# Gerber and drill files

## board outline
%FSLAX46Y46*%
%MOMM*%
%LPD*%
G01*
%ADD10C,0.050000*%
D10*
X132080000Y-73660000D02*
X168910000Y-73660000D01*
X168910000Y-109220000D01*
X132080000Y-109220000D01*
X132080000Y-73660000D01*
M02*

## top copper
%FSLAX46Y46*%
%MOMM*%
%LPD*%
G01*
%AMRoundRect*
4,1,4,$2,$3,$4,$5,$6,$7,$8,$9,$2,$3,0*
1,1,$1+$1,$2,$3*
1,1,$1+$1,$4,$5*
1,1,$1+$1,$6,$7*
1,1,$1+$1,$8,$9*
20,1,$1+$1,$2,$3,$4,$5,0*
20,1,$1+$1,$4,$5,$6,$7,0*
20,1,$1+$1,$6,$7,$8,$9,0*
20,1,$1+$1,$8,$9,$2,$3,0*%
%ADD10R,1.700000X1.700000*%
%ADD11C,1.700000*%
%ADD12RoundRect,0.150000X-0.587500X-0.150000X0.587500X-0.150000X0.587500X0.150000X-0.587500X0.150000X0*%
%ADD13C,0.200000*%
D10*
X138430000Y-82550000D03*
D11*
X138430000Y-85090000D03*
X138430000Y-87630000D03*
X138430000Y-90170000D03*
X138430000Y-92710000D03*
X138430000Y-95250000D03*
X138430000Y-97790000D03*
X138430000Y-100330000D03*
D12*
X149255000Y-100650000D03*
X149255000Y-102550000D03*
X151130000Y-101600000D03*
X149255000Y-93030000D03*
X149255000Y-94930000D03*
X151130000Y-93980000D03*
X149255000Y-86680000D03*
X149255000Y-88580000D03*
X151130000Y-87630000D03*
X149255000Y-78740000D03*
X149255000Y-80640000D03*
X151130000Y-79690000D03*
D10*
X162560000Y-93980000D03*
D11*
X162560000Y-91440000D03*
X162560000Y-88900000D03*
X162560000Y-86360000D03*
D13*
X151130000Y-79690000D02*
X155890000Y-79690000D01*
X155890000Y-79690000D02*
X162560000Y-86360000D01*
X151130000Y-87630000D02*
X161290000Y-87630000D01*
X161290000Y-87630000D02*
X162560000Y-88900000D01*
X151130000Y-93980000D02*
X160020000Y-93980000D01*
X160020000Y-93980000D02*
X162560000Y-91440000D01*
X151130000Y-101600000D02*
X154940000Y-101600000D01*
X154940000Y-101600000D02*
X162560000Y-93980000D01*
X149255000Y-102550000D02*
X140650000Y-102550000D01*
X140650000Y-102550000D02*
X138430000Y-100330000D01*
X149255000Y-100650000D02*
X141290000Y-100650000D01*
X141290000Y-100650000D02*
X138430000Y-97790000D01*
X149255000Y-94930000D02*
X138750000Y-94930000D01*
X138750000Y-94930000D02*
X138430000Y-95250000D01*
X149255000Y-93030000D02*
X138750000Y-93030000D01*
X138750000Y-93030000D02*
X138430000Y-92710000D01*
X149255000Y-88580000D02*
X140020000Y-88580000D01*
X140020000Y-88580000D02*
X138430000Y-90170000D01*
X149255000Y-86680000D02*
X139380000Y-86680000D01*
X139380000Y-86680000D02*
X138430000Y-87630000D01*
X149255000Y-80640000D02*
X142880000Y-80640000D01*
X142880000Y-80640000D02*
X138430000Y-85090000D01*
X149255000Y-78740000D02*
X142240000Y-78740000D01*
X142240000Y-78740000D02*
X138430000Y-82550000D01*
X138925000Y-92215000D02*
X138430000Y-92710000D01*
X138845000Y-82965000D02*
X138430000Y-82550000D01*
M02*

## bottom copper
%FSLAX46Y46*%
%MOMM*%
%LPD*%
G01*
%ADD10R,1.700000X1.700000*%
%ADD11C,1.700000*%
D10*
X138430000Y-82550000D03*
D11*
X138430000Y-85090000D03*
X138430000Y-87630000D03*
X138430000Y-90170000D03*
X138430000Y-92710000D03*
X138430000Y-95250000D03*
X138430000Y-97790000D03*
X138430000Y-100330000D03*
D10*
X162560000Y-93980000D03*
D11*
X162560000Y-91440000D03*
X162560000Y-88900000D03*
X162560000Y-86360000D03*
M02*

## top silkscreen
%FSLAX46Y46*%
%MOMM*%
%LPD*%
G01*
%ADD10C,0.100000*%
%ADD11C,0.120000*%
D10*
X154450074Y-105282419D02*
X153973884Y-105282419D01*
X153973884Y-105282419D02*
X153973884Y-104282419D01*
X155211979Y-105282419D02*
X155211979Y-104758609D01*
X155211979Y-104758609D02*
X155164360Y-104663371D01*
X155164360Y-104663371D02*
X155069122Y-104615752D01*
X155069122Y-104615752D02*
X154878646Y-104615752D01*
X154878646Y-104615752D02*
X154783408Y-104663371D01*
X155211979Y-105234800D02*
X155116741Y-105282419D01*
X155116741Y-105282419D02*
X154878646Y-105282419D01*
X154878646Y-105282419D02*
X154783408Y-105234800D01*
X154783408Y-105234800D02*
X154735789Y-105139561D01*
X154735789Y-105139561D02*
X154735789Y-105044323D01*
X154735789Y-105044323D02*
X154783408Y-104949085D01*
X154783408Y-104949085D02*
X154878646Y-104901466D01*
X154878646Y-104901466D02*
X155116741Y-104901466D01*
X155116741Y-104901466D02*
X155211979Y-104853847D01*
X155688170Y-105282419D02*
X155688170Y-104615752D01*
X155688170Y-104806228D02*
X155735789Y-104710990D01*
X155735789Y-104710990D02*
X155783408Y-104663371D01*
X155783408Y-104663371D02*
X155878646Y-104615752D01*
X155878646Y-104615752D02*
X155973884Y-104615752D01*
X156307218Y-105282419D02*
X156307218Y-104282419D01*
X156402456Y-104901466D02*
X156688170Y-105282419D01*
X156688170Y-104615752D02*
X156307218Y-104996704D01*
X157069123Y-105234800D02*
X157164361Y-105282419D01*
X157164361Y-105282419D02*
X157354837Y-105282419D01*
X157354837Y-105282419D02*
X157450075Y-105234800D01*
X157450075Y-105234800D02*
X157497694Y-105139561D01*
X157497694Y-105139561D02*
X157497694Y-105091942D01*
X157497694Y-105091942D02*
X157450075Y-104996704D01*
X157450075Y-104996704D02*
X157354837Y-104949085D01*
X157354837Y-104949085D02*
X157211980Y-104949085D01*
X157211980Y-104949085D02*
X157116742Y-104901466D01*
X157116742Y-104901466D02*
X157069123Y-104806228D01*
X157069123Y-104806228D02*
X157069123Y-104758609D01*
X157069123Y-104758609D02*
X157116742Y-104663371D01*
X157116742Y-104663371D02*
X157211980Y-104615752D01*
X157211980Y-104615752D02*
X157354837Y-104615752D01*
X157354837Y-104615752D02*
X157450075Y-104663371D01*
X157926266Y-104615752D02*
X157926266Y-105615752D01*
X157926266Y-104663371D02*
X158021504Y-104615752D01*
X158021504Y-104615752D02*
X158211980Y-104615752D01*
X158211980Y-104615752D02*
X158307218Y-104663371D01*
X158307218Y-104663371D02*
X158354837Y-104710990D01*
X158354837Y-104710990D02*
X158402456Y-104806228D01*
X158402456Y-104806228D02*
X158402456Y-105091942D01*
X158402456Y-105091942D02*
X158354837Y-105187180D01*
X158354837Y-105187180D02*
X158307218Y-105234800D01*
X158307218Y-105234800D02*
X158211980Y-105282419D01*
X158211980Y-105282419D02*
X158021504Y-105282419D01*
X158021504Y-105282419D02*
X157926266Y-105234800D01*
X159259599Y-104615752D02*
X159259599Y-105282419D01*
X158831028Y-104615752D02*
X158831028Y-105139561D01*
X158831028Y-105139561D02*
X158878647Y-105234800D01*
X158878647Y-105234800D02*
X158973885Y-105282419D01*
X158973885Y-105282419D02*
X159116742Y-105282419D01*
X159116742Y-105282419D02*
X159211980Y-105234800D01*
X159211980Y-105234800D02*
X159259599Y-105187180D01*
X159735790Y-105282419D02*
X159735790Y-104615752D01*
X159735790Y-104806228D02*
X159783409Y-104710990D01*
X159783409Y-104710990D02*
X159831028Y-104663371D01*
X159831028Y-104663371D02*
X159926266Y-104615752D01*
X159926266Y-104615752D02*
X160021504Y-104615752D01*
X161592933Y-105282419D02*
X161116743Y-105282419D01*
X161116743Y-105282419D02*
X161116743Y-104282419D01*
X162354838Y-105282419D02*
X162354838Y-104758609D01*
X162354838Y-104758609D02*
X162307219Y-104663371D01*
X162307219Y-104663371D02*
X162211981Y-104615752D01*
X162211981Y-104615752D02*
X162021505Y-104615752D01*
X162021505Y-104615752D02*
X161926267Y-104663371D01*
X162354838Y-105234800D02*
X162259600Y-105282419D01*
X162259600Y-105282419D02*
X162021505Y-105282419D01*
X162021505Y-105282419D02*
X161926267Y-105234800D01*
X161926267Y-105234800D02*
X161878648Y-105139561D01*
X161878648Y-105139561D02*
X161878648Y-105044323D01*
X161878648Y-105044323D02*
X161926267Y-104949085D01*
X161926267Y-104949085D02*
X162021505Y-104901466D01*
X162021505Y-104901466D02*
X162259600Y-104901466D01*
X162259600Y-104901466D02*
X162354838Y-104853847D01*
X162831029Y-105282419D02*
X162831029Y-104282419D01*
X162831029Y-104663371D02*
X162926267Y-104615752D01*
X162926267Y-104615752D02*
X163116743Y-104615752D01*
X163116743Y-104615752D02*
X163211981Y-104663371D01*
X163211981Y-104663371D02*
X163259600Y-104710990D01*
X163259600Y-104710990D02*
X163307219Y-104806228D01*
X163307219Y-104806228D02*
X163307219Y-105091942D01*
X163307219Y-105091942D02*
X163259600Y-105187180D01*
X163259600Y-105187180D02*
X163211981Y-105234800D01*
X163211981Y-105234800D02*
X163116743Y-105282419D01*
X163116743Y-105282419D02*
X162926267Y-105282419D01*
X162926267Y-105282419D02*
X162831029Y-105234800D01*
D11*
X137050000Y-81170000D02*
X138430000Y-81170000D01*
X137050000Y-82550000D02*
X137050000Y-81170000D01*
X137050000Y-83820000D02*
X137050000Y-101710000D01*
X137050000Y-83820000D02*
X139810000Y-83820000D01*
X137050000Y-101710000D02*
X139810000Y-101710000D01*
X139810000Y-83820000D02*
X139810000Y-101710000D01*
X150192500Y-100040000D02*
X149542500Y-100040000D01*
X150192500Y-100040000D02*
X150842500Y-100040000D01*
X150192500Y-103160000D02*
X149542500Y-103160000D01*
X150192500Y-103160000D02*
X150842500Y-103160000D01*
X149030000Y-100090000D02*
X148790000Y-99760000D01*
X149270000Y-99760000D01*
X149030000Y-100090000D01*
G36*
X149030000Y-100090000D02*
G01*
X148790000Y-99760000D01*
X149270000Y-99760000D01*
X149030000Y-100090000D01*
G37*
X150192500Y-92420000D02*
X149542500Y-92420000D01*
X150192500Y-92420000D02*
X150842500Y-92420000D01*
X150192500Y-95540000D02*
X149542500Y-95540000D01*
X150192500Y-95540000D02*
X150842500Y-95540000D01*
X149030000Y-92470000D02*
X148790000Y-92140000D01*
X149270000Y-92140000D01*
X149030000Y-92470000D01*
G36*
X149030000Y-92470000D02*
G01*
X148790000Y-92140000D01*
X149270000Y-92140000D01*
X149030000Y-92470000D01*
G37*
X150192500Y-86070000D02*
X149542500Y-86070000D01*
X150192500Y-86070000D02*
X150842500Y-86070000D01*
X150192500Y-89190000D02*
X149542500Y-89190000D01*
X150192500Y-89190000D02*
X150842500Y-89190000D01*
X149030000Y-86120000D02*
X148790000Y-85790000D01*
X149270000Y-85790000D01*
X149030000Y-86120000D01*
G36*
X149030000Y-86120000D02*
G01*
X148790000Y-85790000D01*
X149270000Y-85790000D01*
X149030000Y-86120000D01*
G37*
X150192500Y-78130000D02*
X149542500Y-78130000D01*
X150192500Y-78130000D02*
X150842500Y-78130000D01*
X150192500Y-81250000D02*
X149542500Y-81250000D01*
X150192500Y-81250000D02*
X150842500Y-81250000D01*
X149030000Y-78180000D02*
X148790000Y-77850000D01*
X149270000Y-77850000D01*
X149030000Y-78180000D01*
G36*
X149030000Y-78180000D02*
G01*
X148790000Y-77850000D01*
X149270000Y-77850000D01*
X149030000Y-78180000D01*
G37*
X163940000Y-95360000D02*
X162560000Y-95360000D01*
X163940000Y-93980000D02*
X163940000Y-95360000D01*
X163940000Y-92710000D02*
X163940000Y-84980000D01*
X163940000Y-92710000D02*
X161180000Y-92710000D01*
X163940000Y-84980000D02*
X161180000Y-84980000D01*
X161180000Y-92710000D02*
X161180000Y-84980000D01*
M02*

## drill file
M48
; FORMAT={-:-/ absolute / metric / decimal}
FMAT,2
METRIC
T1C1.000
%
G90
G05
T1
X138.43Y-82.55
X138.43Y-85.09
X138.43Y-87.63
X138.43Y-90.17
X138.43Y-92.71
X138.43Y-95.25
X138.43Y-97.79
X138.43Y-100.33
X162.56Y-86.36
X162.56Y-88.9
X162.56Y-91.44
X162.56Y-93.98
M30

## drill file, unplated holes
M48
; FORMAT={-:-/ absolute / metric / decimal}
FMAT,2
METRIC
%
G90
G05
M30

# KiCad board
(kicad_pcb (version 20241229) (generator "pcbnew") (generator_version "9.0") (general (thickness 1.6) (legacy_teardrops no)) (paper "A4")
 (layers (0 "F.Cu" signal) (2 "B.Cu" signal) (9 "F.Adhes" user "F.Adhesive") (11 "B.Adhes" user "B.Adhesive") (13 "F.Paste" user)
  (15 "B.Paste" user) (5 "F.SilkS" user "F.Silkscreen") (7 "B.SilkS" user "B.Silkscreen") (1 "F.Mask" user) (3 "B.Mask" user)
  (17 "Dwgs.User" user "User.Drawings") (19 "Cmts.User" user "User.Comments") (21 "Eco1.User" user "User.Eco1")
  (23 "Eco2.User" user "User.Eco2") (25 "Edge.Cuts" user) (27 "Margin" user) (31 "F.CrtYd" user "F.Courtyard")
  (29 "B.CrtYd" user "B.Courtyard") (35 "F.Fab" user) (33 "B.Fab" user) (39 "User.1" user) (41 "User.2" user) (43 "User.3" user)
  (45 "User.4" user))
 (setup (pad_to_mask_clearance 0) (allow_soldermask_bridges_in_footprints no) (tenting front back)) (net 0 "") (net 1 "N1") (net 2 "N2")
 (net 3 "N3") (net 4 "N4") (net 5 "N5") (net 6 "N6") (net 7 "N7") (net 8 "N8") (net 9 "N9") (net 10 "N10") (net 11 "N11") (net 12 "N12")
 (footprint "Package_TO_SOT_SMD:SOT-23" (layer "F.Cu") (at 150.1925 87.63)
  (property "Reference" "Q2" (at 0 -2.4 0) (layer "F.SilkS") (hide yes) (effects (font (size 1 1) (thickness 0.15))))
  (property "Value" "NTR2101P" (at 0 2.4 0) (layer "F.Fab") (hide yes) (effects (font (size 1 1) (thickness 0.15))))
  (fp_line (start 0 -1.56) (end -0.65 -1.56) (stroke (width 0.12) (type solid)) (layer "F.SilkS"))
  (fp_line (start 0 -1.56) (end 0.65 -1.56) (stroke (width 0.12) (type solid)) (layer "F.SilkS"))
  (fp_line (start 0 1.56) (end -0.65 1.56) (stroke (width 0.12) (type solid)) (layer "F.SilkS"))
  (fp_line (start 0 1.56) (end 0.65 1.56) (stroke (width 0.12) (type solid)) (layer "F.SilkS"))
  (fp_poly (pts (xy -1.1625 -1.51) (xy -1.4025 -1.84) (xy -0.9225 -1.84)) (stroke (width 0.12) (type solid)) (fill yes) (layer "F.SilkS"))
  (pad "1" smd roundrect (at -0.9375 -0.95) (size 1.475 0.6) (layers "F.Cu" "F.Mask" "F.Paste") (roundrect_rratio 0.25) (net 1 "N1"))
  (pad "2" smd roundrect (at -0.9375 0.95) (size 1.475 0.6) (layers "F.Cu" "F.Mask" "F.Paste") (roundrect_rratio 0.25) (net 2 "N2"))
  (pad "3" smd roundrect (at 0.9375 0) (size 1.475 0.6) (layers "F.Cu" "F.Mask" "F.Paste") (roundrect_rratio 0.25) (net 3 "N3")))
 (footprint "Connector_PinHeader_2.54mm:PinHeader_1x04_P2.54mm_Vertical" (layer "F.Cu") (at 162.56 93.98 180)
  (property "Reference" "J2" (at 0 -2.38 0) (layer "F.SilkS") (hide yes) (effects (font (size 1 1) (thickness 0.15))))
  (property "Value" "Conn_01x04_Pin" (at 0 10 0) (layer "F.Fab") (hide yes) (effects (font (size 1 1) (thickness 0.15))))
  (fp_line (start 1.38 1.27) (end 1.38 9) (stroke (width 0.12) (type solid)) (layer "F.SilkS"))
  (fp_line (start -1.38 9) (end 1.38 9) (stroke (width 0.12) (type solid)) (layer "F.SilkS"))
  (fp_line (start -1.38 1.27) (end 1.38 1.27) (stroke (width 0.12) (type solid)) (layer "F.SilkS"))
  (fp_line (start -1.38 1.27) (end -1.38 9) (stroke (width 0.12) (type solid)) (layer "F.SilkS"))
  (fp_line (start -1.38 0) (end -1.38 -1.38) (stroke (width 0.12) (type solid)) (layer "F.SilkS"))
  (fp_line (start -1.38 -1.38) (end 0 -1.38) (stroke (width 0.12) (type solid)) (layer "F.SilkS"))
  (pad "1" thru_hole rect (at 0 0 180) (size 1.7 1.7) (drill 1) (layers "*.Cu" "*.Mask") (remove_unused_layers no) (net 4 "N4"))
  (pad "2" thru_hole circle (at 0 2.54 180) (size 1.7 1.7) (drill 1) (layers "*.Cu" "*.Mask") (remove_unused_layers no) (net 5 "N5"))
  (pad "3" thru_hole circle (at 0 5.08 180) (size 1.7 1.7) (drill 1) (layers "*.Cu" "*.Mask") (remove_unused_layers no) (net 3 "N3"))
  (pad "4" thru_hole circle (at 0 7.62 180) (size 1.7 1.7) (drill 1) (layers "*.Cu" "*.Mask") (remove_unused_layers no) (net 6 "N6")))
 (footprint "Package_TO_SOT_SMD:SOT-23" (layer "F.Cu") (at 150.1925 79.69)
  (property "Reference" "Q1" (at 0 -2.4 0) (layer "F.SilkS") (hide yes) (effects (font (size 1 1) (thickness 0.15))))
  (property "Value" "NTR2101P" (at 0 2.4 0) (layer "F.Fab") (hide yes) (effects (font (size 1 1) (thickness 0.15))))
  (fp_line (start 0 -1.56) (end -0.65 -1.56) (stroke (width 0.12) (type solid)) (layer "F.SilkS"))
  (fp_line (start 0 -1.56) (end 0.65 -1.56) (stroke (width 0.12) (type solid)) (layer "F.SilkS"))
  (fp_line (start 0 1.56) (end -0.65 1.56) (stroke (width 0.12) (type solid)) (layer "F.SilkS"))
  (fp_line (start 0 1.56) (end 0.65 1.56) (stroke (width 0.12) (type solid)) (layer "F.SilkS"))
  (fp_poly (pts (xy -1.1625 -1.51) (xy -1.4025 -1.84) (xy -0.9225 -1.84)) (stroke (width 0.12) (type solid)) (fill yes) (layer "F.SilkS"))
  (pad "1" smd roundrect (at -0.9375 -0.95) (size 1.475 0.6) (layers "F.Cu" "F.Mask" "F.Paste") (roundrect_rratio 0.25) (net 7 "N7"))
  (pad "2" smd roundrect (at -0.9375 0.95) (size 1.475 0.6) (layers "F.Cu" "F.Mask" "F.Paste") (roundrect_rratio 0.25) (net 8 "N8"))
  (pad "3" smd roundrect (at 0.9375 0) (size 1.475 0.6) (layers "F.Cu" "F.Mask" "F.Paste") (roundrect_rratio 0.25) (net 6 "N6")))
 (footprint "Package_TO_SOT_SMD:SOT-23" (layer "F.Cu") (at 150.1925 101.6)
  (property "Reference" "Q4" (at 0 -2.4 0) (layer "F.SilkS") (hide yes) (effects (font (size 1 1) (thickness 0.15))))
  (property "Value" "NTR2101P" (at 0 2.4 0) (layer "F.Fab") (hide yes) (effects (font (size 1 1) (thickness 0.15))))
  (fp_line (start 0 -1.56) (end -0.65 -1.56) (stroke (width 0.12) (type solid)) (layer "F.SilkS"))
  (fp_line (start 0 -1.56) (end 0.65 -1.56) (stroke (width 0.12) (type solid)) (layer "F.SilkS"))
  (fp_line (start 0 1.56) (end -0.65 1.56) (stroke (width 0.12) (type solid)) (layer "F.SilkS"))
  (fp_line (start 0 1.56) (end 0.65 1.56) (stroke (width 0.12) (type solid)) (layer "F.SilkS"))
  (fp_poly (pts (xy -1.1625 -1.51) (xy -1.4025 -1.84) (xy -0.9225 -1.84)) (stroke (width 0.12) (type solid)) (fill yes) (layer "F.SilkS"))
  (pad "1" smd roundrect (at -0.9375 -0.95) (size 1.475 0.6) (layers "F.Cu" "F.Mask" "F.Paste") (roundrect_rratio 0.25) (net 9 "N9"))
  (pad "2" smd roundrect (at -0.9375 0.95) (size 1.475 0.6) (layers "F.Cu" "F.Mask" "F.Paste") (roundrect_rratio 0.25) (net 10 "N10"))
  (pad "3" smd roundrect (at 0.9375 0) (size 1.475 0.6) (layers "F.Cu" "F.Mask" "F.Paste") (roundrect_rratio 0.25) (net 4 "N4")))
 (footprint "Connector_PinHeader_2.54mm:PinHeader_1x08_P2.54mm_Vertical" (layer "F.Cu") (at 138.43 82.55)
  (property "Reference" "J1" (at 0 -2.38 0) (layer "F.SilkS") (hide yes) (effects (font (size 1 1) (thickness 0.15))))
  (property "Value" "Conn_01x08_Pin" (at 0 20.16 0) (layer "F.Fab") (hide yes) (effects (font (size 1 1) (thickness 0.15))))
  (fp_line (start -1.38 -1.38) (end 0 -1.38) (stroke (width 0.12) (type solid)) (layer "F.SilkS"))
  (fp_line (start -1.38 0) (end -1.38 -1.38) (stroke (width 0.12) (type solid)) (layer "F.SilkS"))
  (fp_line (start -1.38 1.27) (end -1.38 19.16) (stroke (width 0.12) (type solid)) (layer "F.SilkS"))
  (fp_line (start -1.38 1.27) (end 1.38 1.27) (stroke (width 0.12) (type solid)) (layer "F.SilkS"))
  (fp_line (start -1.38 19.16) (end 1.38 19.16) (stroke (width 0.12) (type solid)) (layer "F.SilkS"))
  (fp_line (start 1.38 1.27) (end 1.38 19.16) (stroke (width 0.12) (type solid)) (layer "F.SilkS"))
  (pad "1" thru_hole rect (at 0 0) (size 1.7 1.7) (drill 1) (layers "*.Cu" "*.Mask") (remove_unused_layers no) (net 7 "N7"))
  (pad "2" thru_hole circle (at 0 2.54) (size 1.7 1.7) (drill 1) (layers "*.Cu" "*.Mask") (remove_unused_layers no) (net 8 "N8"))
  (pad "3" thru_hole circle (at 0 5.08) (size 1.7 1.7) (drill 1) (layers "*.Cu" "*.Mask") (remove_unused_layers no) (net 1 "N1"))
  (pad "4" thru_hole circle (at 0 7.62) (size 1.7 1.7) (drill 1) (layers "*.Cu" "*.Mask") (remove_unused_layers no) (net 2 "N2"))
  (pad "5" thru_hole circle (at 0 10.16) (size 1.7 1.7) (drill 1) (layers "*.Cu" "*.Mask") (remove_unused_layers no) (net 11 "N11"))
  (pad "6" thru_hole circle (at 0 12.7) (size 1.7 1.7) (drill 1) (layers "*.Cu" "*.Mask") (remove_unused_layers no) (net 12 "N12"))
  (pad "7" thru_hole circle (at 0 15.24) (size 1.7 1.7) (drill 1) (layers "*.Cu" "*.Mask") (remove_unused_layers no) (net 9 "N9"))
  (pad "8" thru_hole circle (at 0 17.78) (size 1.7 1.7) (drill 1) (layers "*.Cu" "*.Mask") (remove_unused_layers no) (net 10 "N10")))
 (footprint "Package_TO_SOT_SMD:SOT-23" (layer "F.Cu") (at 150.1925 93.98)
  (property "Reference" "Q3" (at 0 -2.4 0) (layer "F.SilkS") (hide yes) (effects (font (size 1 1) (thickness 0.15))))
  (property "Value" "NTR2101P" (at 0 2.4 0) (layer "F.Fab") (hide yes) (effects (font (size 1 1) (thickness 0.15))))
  (fp_line (start 0 -1.56) (end -0.65 -1.56) (stroke (width 0.12) (type solid)) (layer "F.SilkS"))
  (fp_line (start 0 -1.56) (end 0.65 -1.56) (stroke (width 0.12) (type solid)) (layer "F.SilkS"))
  (fp_line (start 0 1.56) (end -0.65 1.56) (stroke (width 0.12) (type solid)) (layer "F.SilkS"))
  (fp_line (start 0 1.56) (end 0.65 1.56) (stroke (width 0.12) (type solid)) (layer "F.SilkS"))
  (fp_poly (pts (xy -1.1625 -1.51) (xy -1.4025 -1.84) (xy -0.9225 -1.84)) (stroke (width 0.12) (type solid)) (fill yes) (layer "F.SilkS"))
  (pad "1" smd roundrect (at -0.9375 -0.95) (size 1.475 0.6) (layers "F.Cu" "F.Mask" "F.Paste") (roundrect_rratio 0.25) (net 11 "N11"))
  (pad "2" smd roundrect (at -0.9375 0.95) (size 1.475 0.6) (layers "F.Cu" "F.Mask" "F.Paste") (roundrect_rratio 0.25) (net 12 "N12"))
  (pad "3" smd roundrect (at 0.9375 0) (size 1.475 0.6) (layers "F.Cu" "F.Mask" "F.Paste") (roundrect_rratio 0.25) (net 5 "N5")))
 (gr_rect (start 132.08 73.66) (end 168.91 109.22) (stroke (width 0.05) (type default)) (fill no) (layer "Edge.Cuts"))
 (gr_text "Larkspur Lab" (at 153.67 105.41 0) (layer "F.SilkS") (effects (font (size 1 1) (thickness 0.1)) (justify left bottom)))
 (segment (start 149.255 80.64) (end 142.88 80.64) (width 0.2) (layer "F.Cu") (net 8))
 (segment (start 142.88 80.64) (end 138.43 85.09) (width 0.2) (layer "F.Cu") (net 8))
 (segment (start 155.89 79.69) (end 162.56 86.36) (width 0.2) (layer "F.Cu") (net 6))
 (segment (start 151.13 79.69) (end 155.89 79.69) (width 0.2) (layer "F.Cu") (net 6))
 (segment (start 142.24 78.74) (end 138.43 82.55) (width 0.2) (layer "F.Cu") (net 7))
 (segment (start 138.845 82.965) (end 138.43 82.55) (width 0.2) (layer "F.Cu") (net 7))
 (segment (start 149.255 78.74) (end 142.24 78.74) (width 0.2) (layer "F.Cu") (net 7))
 (segment (start 151.13 87.63) (end 161.29 87.63) (width 0.2) (layer "F.Cu") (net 3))
 (segment (start 161.29 87.63) (end 162.56 88.9) (width 0.2) (layer "F.Cu") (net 3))
 (segment (start 140.02 88.58) (end 138.43 90.17) (width 0.2) (layer "F.Cu") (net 2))
 (segment (start 149.255 88.58) (end 140.02 88.58) (width 0.2) (layer "F.Cu") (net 2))
 (segment (start 149.255 86.68) (end 139.38 86.68) (width 0.2) (layer "F.Cu") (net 1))
 (segment (start 139.38 86.68) (end 138.43 87.63) (width 0.2) (layer "F.Cu") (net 1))
 (segment (start 149.255 93.03) (end 138.75 93.03) (width 0.2) (layer "F.Cu") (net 11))
 (segment (start 138.925 92.215) (end 138.43 92.71) (width 0.2) (layer "F.Cu") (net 11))
 (segment (start 138.75 93.03) (end 138.43 92.71) (width 0.2) (layer "F.Cu") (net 11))
 (segment (start 149.255 94.93) (end 138.75 94.93) (width 0.2) (layer "F.Cu") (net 12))
 (segment (start 138.75 94.93) (end 138.43 95.25) (width 0.2) (layer "F.Cu") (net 12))
 (segment (start 160.02 93.98) (end 162.56 91.44) (width 0.2) (layer "F.Cu") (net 5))
 (segment (start 151.13 93.98) (end 160.02 93.98) (width 0.2) (layer "F.Cu") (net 5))
 (segment (start 149.255 102.55) (end 140.65 102.55) (width 0.2) (layer "F.Cu") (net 10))
 (segment (start 140.65 102.55) (end 138.43 100.33) (width 0.2) (layer "F.Cu") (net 10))
 (segment (start 151.13 101.6) (end 154.94 101.6) (width 0.2) (layer "F.Cu") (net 4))
 (segment (start 154.94 101.6) (end 162.56 93.98) (width 0.2) (layer "F.Cu") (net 4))
 (segment (start 141.29 100.65) (end 138.43 97.79) (width 0.2) (layer "F.Cu") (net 9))
 (segment (start 149.255 100.65) (end 141.29 100.65) (width 0.2) (layer "F.Cu") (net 9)))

